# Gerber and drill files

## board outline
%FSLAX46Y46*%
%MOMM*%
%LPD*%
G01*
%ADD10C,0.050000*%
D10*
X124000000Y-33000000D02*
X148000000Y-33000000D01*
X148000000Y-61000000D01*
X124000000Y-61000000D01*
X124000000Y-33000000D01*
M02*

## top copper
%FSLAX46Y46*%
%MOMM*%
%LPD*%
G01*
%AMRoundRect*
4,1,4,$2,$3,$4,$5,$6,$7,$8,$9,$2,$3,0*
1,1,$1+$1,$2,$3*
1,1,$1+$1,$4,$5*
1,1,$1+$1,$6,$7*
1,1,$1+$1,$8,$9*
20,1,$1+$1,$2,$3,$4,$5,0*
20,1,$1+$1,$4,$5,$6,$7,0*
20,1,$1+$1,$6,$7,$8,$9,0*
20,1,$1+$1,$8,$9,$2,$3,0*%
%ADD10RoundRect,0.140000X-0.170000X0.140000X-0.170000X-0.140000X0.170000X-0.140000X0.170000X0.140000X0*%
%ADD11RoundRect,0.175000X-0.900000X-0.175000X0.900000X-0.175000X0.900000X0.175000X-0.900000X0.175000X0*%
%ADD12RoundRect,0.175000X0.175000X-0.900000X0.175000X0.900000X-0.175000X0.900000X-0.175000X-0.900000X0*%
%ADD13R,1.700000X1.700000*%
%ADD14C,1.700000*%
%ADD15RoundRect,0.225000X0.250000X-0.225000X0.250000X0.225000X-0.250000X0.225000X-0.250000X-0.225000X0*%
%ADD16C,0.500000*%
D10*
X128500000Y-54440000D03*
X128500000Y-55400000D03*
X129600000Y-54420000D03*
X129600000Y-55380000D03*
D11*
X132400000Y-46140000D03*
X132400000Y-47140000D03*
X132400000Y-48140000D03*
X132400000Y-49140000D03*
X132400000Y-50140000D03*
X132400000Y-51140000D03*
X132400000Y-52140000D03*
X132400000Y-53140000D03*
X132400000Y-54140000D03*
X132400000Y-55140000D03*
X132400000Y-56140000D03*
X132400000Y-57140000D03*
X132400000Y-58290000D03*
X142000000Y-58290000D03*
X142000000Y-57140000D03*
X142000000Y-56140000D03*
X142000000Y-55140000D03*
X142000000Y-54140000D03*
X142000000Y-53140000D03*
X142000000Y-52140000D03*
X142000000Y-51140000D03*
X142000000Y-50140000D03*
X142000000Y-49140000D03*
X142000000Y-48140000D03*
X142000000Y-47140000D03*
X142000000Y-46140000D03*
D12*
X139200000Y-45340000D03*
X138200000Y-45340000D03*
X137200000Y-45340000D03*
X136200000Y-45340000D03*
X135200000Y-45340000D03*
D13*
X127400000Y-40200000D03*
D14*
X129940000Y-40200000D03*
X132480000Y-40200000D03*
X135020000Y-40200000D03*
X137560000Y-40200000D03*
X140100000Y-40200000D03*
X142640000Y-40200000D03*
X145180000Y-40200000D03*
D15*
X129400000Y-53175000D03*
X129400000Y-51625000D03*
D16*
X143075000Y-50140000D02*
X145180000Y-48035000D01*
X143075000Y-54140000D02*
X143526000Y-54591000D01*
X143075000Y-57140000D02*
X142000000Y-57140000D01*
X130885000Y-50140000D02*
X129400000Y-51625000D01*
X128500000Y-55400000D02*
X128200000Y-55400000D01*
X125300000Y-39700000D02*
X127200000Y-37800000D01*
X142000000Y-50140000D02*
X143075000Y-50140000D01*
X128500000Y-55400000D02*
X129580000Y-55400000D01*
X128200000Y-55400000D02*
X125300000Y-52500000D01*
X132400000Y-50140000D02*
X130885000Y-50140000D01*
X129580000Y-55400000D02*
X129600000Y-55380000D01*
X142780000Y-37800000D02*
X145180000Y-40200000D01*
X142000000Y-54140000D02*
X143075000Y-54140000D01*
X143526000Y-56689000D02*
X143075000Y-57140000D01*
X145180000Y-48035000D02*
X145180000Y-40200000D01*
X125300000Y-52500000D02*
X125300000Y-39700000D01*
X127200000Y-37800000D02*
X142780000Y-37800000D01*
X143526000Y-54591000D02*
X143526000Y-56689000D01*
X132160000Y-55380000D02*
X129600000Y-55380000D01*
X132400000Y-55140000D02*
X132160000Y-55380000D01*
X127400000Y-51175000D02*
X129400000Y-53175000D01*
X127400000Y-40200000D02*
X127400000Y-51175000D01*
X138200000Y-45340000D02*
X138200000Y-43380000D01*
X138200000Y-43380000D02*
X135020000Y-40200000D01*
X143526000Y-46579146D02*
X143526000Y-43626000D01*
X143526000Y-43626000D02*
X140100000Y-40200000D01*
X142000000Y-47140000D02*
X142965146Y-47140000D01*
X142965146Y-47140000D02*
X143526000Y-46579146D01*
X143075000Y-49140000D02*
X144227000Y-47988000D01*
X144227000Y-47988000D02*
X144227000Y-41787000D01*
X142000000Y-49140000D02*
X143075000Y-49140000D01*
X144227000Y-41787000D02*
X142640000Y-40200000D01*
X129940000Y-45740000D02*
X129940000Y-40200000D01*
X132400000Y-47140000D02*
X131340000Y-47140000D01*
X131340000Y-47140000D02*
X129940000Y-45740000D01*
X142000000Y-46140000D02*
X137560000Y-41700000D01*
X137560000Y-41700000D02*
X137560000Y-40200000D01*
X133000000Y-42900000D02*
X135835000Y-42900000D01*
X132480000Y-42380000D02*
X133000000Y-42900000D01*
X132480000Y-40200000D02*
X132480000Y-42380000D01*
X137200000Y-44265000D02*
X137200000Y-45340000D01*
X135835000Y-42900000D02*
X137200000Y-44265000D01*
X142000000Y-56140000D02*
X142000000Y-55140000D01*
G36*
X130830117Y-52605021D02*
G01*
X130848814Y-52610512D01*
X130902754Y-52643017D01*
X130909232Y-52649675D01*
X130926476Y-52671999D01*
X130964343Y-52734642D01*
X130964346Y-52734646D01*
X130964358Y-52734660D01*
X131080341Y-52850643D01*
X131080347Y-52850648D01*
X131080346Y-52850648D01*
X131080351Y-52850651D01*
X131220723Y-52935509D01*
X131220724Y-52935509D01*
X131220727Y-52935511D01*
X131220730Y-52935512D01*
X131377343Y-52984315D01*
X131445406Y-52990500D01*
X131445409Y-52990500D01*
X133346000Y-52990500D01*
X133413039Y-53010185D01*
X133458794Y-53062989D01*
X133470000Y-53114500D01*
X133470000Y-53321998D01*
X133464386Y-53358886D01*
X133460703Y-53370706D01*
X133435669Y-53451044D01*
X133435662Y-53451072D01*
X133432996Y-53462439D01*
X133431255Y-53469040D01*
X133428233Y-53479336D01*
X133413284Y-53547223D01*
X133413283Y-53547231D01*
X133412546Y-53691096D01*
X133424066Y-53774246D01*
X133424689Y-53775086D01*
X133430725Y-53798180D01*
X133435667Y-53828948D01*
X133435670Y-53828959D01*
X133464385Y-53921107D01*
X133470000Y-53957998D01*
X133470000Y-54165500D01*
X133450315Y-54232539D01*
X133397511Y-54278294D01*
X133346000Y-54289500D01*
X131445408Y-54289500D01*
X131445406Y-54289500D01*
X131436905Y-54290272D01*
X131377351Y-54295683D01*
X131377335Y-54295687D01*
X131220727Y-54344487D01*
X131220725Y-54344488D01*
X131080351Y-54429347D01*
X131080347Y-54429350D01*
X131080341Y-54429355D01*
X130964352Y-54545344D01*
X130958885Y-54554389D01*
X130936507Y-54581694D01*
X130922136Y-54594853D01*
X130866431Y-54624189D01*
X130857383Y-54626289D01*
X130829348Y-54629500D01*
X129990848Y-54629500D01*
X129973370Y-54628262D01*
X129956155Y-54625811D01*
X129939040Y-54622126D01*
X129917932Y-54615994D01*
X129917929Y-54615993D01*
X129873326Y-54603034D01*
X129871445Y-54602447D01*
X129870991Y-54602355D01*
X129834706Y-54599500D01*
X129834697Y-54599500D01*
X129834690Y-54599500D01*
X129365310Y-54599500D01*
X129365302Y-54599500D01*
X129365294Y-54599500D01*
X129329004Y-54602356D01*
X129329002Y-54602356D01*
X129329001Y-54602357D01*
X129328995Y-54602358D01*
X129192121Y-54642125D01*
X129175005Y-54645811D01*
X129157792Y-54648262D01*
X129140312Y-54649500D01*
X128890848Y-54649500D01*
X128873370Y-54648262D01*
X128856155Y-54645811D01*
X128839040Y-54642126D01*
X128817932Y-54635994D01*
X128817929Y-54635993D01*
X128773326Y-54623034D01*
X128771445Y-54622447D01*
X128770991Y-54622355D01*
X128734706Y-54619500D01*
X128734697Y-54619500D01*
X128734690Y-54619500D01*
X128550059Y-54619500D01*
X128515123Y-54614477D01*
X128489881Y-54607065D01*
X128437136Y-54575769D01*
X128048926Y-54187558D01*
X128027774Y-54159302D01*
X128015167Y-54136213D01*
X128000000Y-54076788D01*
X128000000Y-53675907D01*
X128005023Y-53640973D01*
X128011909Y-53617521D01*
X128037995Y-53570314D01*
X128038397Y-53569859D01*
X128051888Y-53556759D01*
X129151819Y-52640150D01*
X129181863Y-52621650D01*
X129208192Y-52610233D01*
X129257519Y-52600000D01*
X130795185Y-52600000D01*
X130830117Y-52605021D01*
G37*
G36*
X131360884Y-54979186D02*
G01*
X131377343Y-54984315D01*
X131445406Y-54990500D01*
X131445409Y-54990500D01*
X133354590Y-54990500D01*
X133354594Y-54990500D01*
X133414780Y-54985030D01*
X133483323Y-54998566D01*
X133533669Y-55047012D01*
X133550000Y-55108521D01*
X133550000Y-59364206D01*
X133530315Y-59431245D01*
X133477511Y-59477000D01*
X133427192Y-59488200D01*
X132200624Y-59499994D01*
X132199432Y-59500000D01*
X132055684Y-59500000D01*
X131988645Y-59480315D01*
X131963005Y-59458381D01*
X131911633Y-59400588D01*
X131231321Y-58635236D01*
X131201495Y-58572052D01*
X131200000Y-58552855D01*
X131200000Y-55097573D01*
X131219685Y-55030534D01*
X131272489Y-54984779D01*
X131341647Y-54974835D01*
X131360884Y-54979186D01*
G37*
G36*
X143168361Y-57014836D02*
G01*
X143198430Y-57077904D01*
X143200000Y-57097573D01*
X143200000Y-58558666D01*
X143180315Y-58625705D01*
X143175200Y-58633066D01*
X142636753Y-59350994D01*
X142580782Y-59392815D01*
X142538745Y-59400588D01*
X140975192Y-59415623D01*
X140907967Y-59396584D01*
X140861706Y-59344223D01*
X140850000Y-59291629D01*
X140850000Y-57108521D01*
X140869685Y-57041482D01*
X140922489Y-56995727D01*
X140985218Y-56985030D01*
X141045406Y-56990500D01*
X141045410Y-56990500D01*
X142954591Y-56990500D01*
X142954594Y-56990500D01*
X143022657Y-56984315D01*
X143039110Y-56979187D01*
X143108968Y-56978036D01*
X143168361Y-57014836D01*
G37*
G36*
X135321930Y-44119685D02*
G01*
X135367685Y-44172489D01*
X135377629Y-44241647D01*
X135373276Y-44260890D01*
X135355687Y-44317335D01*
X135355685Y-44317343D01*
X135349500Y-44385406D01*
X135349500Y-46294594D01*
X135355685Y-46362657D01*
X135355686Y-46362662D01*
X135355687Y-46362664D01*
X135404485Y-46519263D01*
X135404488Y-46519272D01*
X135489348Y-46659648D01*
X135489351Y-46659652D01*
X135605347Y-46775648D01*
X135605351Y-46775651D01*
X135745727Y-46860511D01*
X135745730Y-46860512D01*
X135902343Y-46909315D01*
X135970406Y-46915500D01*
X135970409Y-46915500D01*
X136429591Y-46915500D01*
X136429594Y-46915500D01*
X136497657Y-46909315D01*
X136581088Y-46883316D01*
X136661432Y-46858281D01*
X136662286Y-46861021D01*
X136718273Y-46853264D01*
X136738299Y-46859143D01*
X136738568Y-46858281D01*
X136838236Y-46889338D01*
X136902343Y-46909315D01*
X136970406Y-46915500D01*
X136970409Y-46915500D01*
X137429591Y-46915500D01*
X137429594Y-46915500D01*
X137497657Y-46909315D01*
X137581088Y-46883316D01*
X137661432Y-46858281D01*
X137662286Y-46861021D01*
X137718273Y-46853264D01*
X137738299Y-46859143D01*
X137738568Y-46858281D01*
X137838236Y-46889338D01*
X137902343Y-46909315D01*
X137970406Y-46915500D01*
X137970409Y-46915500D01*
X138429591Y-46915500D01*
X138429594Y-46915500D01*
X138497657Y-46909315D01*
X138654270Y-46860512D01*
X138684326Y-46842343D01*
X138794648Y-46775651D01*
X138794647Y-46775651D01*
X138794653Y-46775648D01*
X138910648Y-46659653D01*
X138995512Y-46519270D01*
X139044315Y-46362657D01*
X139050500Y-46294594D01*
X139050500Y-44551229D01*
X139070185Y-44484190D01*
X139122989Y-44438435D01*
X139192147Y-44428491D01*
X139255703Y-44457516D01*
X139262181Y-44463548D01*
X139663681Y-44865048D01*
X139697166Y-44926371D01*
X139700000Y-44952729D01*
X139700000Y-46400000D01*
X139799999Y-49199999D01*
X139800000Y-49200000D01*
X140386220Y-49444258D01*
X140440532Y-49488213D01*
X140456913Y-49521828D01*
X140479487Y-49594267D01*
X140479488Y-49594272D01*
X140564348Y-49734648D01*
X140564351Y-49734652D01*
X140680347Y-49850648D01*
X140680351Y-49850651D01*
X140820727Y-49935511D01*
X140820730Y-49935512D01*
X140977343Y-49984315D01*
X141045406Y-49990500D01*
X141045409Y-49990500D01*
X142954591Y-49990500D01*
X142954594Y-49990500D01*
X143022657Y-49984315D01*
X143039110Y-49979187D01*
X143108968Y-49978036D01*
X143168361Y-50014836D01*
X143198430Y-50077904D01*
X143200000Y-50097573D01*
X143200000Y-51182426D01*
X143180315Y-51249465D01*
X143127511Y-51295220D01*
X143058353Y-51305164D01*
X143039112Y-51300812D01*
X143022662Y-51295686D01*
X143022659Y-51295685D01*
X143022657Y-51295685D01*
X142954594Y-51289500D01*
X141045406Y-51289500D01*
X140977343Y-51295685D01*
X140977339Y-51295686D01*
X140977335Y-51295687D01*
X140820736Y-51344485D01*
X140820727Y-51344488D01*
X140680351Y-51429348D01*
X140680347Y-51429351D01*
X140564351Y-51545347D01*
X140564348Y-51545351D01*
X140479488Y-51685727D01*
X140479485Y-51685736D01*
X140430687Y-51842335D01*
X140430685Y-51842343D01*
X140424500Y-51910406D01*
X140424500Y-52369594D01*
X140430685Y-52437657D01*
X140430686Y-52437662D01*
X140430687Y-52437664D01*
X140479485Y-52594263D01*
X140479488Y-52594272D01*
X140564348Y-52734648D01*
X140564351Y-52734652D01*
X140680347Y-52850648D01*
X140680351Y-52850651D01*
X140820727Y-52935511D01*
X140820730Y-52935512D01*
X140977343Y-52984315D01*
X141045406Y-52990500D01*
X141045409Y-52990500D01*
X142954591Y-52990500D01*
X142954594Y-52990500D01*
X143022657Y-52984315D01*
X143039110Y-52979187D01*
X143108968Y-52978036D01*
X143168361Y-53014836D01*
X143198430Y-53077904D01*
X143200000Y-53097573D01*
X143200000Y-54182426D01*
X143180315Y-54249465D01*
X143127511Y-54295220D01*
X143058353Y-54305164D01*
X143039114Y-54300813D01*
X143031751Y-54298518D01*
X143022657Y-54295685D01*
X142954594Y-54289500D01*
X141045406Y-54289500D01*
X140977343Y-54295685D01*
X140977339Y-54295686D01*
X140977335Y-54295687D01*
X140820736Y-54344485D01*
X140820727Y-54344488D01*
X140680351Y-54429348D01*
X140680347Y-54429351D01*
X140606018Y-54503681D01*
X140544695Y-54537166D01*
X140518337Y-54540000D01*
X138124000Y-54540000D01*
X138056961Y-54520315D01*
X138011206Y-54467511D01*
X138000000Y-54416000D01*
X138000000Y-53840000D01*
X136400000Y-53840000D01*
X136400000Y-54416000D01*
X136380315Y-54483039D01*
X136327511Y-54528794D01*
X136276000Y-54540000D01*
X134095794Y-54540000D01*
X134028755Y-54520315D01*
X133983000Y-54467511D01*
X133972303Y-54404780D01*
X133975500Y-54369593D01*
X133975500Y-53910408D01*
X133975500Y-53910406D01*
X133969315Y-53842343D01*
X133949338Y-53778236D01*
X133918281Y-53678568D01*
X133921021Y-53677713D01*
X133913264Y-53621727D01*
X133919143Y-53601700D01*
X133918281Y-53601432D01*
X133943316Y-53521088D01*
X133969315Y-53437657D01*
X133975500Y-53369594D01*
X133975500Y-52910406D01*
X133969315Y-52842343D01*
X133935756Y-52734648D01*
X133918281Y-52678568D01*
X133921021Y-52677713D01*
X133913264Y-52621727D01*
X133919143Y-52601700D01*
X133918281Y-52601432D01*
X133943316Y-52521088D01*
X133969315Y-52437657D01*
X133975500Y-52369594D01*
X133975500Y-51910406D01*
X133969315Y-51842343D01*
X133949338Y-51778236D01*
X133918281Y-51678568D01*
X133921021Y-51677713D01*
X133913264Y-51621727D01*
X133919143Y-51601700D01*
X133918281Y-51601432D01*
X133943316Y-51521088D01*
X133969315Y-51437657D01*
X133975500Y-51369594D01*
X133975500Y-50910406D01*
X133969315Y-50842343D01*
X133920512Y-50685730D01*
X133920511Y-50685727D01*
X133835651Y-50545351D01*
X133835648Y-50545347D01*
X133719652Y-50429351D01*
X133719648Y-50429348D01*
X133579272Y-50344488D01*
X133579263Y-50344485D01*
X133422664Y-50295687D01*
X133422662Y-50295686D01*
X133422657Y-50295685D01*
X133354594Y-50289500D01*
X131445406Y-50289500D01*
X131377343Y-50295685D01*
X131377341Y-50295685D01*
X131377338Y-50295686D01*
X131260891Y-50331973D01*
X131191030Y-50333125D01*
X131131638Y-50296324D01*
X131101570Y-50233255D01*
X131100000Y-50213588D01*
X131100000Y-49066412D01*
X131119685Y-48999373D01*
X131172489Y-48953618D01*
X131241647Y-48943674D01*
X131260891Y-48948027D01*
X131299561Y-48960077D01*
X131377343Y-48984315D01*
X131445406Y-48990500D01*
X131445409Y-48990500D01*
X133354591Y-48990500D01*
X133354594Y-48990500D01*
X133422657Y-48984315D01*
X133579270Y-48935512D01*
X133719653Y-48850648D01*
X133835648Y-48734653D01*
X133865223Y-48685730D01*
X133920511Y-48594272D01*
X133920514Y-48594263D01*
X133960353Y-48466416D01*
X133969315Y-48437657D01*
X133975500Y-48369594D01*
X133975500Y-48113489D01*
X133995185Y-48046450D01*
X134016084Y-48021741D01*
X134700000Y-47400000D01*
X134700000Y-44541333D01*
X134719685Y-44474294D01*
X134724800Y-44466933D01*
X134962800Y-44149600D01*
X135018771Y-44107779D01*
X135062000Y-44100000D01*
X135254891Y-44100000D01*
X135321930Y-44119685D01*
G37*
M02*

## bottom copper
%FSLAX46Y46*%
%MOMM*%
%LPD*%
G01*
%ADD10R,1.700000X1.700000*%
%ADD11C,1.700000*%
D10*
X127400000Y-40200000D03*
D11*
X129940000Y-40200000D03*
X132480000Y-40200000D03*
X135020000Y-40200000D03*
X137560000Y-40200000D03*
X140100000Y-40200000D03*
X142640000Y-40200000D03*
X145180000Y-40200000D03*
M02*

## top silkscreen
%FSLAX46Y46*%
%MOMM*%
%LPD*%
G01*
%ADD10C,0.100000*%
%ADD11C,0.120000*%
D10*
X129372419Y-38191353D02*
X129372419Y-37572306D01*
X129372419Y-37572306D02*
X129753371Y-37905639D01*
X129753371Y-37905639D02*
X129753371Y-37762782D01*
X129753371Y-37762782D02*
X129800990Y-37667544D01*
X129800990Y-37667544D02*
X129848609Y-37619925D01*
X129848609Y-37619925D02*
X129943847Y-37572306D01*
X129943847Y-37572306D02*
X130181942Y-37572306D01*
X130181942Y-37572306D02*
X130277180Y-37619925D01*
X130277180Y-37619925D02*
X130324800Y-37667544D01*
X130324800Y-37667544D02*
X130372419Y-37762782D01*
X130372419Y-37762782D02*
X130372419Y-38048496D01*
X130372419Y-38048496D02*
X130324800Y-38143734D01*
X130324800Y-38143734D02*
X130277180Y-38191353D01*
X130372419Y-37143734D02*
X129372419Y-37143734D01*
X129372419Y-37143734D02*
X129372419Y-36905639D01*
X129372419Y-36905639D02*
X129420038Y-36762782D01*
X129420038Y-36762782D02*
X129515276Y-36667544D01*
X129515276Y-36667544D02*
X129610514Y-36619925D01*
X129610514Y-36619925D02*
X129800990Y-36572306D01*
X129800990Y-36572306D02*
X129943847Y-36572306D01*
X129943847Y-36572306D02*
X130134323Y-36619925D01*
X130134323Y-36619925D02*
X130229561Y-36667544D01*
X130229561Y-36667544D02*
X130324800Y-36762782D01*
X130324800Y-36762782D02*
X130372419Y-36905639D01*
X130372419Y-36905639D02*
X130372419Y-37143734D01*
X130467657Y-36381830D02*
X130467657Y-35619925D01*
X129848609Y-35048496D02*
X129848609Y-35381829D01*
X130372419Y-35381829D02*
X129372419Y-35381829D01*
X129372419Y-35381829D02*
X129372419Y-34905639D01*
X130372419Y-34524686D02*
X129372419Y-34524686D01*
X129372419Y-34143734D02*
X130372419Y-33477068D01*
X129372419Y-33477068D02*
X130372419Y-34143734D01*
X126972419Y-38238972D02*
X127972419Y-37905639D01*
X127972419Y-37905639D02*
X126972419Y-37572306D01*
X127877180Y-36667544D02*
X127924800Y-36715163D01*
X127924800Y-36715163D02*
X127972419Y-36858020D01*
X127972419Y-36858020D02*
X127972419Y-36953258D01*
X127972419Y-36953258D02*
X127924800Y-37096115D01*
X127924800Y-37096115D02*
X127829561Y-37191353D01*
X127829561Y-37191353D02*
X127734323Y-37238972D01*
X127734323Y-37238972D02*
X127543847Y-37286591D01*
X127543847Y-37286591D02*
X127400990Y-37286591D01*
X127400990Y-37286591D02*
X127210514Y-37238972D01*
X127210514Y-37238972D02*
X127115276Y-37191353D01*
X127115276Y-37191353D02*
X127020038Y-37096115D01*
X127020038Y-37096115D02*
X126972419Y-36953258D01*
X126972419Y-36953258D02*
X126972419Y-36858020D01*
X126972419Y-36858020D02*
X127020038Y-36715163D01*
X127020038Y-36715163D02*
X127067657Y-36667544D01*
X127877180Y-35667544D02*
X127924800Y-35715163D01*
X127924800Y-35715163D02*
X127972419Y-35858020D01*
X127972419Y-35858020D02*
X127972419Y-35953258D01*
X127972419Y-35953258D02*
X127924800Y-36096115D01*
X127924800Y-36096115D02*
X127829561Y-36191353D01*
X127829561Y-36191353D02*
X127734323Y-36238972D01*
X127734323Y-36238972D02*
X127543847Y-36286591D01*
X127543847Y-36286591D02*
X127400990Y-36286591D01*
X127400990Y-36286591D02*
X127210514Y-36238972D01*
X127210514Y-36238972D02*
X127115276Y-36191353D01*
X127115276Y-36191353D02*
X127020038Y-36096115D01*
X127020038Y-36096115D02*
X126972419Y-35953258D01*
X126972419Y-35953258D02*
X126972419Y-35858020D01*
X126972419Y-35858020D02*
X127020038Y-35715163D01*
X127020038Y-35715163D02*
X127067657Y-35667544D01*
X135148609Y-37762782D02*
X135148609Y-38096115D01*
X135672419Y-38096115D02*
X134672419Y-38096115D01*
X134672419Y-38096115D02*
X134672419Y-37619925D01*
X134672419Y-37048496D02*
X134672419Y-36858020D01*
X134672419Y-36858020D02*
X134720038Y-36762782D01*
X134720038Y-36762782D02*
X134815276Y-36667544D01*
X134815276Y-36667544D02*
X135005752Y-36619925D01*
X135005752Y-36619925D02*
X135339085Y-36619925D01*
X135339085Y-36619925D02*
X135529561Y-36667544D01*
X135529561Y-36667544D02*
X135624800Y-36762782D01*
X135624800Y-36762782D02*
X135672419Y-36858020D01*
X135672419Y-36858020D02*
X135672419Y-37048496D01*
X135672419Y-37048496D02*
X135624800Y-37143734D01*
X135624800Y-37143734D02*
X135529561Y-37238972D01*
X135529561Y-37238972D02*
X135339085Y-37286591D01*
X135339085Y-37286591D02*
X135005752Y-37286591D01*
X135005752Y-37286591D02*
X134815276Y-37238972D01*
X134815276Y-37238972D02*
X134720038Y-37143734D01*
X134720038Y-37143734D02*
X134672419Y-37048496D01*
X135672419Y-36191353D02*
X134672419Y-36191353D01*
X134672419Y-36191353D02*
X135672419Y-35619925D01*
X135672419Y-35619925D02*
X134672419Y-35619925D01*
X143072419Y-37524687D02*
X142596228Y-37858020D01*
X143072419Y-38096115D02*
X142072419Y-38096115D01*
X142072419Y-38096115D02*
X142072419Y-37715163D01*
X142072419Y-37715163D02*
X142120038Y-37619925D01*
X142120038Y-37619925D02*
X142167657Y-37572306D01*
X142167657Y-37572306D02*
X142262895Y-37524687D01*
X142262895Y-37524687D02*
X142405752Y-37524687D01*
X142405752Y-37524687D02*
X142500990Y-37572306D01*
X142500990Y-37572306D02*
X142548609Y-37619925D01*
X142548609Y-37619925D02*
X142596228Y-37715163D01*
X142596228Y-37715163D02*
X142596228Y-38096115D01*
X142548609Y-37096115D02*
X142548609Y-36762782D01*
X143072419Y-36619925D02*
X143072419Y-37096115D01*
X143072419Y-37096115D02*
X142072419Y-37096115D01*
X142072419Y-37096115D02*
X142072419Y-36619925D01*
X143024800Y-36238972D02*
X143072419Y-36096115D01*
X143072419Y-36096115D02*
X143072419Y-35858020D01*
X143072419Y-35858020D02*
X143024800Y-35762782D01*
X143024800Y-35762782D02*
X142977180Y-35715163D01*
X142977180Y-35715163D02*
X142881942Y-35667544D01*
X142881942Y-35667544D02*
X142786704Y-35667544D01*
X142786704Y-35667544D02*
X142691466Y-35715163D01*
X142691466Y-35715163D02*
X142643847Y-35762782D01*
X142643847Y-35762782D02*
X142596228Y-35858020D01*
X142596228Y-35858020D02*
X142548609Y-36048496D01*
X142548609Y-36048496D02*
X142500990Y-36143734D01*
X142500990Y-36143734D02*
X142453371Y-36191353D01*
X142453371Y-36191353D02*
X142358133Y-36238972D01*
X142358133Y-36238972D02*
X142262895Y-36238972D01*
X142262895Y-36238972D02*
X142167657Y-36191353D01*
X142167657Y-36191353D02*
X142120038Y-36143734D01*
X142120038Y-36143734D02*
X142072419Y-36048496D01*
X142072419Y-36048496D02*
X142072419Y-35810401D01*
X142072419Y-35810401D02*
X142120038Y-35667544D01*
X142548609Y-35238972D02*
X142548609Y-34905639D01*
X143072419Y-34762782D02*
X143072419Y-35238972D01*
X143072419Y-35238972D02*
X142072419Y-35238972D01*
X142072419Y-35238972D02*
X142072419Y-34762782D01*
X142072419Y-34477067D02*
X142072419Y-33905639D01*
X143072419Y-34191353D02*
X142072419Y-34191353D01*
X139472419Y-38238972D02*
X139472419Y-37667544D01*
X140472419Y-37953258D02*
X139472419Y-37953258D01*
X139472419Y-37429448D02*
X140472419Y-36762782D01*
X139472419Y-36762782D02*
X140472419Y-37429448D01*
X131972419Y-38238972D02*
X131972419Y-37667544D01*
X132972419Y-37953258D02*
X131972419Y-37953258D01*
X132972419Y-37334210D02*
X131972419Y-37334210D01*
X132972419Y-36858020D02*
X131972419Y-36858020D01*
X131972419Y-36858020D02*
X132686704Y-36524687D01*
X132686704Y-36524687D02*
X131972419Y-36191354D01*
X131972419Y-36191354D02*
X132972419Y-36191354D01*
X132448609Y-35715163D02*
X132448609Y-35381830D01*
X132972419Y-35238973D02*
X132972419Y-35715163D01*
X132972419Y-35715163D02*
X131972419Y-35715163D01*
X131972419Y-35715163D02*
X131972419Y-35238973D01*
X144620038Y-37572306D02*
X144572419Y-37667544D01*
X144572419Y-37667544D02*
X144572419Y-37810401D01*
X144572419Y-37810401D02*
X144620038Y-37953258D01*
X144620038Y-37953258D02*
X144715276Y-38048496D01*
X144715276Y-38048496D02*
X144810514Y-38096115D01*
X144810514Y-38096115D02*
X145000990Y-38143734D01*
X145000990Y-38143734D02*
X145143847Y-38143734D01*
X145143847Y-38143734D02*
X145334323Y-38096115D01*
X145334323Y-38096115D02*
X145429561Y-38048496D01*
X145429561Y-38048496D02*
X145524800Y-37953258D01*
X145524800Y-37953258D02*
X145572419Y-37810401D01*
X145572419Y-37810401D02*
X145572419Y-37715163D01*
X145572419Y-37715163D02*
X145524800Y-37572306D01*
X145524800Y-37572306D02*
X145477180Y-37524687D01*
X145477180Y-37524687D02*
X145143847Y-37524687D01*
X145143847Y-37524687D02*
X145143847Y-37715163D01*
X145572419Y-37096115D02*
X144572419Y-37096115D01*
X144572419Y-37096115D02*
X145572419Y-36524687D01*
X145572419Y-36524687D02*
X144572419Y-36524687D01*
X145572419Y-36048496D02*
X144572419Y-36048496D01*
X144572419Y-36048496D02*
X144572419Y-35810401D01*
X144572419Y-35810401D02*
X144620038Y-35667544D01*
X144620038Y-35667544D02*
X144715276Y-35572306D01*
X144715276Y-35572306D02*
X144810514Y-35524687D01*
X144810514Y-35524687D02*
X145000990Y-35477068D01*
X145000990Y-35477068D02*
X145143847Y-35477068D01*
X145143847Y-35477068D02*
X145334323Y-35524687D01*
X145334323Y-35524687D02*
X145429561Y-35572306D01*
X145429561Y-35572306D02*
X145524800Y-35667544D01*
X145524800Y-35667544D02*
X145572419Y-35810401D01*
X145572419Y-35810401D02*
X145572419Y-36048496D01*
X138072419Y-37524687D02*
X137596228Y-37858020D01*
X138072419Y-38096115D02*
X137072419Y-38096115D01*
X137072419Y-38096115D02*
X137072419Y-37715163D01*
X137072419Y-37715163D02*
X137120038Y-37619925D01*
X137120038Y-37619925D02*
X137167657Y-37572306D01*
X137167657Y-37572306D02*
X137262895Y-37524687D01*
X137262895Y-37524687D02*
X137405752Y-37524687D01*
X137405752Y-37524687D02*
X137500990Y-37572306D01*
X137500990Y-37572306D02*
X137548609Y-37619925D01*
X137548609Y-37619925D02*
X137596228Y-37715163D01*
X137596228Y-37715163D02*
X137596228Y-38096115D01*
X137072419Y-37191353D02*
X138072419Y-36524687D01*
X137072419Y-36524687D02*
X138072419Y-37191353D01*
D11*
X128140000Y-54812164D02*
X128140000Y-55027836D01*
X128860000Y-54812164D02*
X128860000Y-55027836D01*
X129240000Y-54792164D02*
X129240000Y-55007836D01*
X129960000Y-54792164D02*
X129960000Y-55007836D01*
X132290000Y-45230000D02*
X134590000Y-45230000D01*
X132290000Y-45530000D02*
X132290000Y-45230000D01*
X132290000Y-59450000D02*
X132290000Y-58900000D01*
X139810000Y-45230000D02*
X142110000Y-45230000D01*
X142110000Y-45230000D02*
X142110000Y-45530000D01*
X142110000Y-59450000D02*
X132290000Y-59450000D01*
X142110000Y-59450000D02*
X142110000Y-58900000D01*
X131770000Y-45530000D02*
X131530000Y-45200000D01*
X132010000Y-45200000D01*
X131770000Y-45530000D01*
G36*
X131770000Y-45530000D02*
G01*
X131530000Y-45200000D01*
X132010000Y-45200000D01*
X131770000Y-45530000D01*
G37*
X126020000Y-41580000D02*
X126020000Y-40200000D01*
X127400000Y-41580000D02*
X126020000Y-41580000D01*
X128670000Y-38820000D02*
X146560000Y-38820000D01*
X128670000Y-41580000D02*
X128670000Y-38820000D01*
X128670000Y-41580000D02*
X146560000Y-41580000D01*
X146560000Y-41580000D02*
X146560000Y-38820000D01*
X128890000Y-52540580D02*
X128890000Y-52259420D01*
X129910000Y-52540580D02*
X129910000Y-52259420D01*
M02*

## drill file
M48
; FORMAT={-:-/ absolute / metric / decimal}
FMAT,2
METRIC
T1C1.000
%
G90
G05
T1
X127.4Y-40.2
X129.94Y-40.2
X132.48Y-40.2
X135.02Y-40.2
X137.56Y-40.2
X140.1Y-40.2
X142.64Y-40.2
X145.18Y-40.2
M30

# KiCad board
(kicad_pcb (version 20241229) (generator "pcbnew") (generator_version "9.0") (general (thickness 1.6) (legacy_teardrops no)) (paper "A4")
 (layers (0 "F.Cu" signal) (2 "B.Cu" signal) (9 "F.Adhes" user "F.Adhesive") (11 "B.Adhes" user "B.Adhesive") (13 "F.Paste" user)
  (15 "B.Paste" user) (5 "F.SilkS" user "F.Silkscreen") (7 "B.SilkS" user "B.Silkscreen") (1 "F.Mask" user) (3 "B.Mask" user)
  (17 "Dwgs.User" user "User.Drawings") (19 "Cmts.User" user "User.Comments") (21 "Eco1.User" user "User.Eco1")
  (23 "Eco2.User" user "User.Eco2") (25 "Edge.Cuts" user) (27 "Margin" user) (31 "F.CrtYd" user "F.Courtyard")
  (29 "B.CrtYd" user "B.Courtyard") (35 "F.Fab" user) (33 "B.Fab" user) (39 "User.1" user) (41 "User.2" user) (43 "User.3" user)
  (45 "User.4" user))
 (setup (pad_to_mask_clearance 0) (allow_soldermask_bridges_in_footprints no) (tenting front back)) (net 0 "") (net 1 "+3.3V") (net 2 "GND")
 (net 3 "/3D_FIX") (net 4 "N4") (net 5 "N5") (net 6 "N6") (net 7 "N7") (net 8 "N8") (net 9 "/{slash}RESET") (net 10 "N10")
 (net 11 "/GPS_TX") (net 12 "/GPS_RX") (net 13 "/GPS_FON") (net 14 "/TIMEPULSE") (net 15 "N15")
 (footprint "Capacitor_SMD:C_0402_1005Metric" (layer "F.Cu") (at 128.5 54.92 -90)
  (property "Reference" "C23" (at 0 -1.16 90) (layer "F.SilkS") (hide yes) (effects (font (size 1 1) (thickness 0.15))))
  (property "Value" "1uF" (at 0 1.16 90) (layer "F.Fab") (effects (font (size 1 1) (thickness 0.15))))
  (fp_line (start -0.107836 0.36) (end 0.107836 0.36) (stroke (width 0.12) (type solid)) (layer "F.SilkS"))
  (fp_line (start -0.107836 -0.36) (end 0.107836 -0.36) (stroke (width 0.12) (type solid)) (layer "F.SilkS"))
  (pad "1" smd roundrect (at -0.48 0 270) (size 0.56 0.62) (layers "F.Cu" "F.Mask" "F.Paste") (roundrect_rratio 0.25) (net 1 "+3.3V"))
  (pad "2" smd roundrect (at 0.48 0 270) (size 0.56 0.62) (layers "F.Cu" "F.Mask" "F.Paste") (roundrect_rratio 0.25) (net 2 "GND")))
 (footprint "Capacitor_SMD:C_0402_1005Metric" (layer "F.Cu") (at 129.6 54.9 -90)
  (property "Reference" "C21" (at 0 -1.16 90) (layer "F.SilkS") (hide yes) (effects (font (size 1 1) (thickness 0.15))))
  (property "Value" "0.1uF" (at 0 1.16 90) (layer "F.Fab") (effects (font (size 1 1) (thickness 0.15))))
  (fp_line (start -0.107836 0.36) (end 0.107836 0.36) (stroke (width 0.12) (type solid)) (layer "F.SilkS"))
  (fp_line (start -0.107836 -0.36) (end 0.107836 -0.36) (stroke (width 0.12) (type solid)) (layer "F.SilkS"))
  (pad "1" smd roundrect (at -0.48 0 270) (size 0.56 0.62) (layers "F.Cu" "F.Mask" "F.Paste") (roundrect_rratio 0.25) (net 1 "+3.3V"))
  (pad "2" smd roundrect (at 0.48 0 270) (size 0.56 0.62) (layers "F.Cu" "F.Mask" "F.Paste") (roundrect_rratio 0.25) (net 2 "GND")))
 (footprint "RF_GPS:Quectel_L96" (layer "F.Cu") (at 137.2 52.34)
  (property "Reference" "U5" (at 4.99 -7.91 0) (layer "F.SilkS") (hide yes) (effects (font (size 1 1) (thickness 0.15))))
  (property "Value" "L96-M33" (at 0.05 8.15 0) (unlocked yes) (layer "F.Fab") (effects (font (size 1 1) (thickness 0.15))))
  (fp_line (start -4.91 -7.11) (end -2.61 -7.11) (stroke (width 0.12) (type default)) (layer "F.SilkS"))
  (fp_line (start -4.91 -6.81) (end -4.91 -7.11) (stroke (width 0.12) (type default)) (layer "F.SilkS"))
  (fp_line (start -4.91 7.11) (end -4.91 6.56) (stroke (width 0.12) (type default)) (layer "F.SilkS"))
  (fp_line (start 2.61 -7.11) (end 4.91 -7.11) (stroke (width 0.12) (type default)) (layer "F.SilkS"))
  (fp_line (start 4.91 -7.11) (end 4.91 -6.81) (stroke (width 0.12) (type default)) (layer "F.SilkS"))
  (fp_line (start 4.91 7.11) (end -4.91 7.11) (stroke (width 0.12) (type default)) (layer "F.SilkS"))
  (fp_line (start 4.91 7.11) (end 4.91 6.56) (stroke (width 0.12) (type default)) (layer "F.SilkS"))
  (fp_poly
   (pts (xy -5.43 -6.81) (xy -5.67 -7.14) (xy -5.19 -7.14) (xy -5.43 -6.81)) (stroke (width 0.12) (type solid)) (fill yes) (layer "F.SilkS"))
  (pad "1" smd roundrect (at -4.8 -6.2) (size 2.15 0.7) (layers "F.Cu" "F.Mask" "F.Paste") (roundrect_rratio 0.25) (thermal_bridge_angle 45))
  (pad "2" smd roundrect (at -4.8 -5.2) (size 2.15 0.7) (layers "F.Cu" "F.Mask" "F.Paste") (roundrect_rratio 0.25) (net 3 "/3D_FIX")
   (thermal_bridge_angle 45))
  (pad "3" smd roundrect (at -4.8 -4.2) (size 2.15 0.7) (layers "F.Cu" "F.Mask" "F.Paste") (roundrect_rratio 0.25) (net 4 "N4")
   (thermal_bridge_angle 45))
  (pad "4" smd roundrect (at -4.8 -3.2) (size 2.15 0.7) (layers "F.Cu" "F.Mask" "F.Paste") (roundrect_rratio 0.25) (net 2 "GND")
   (thermal_bridge_angle 45))
  (pad "5" smd roundrect (at -4.8 -2.2) (size 2.15 0.7) (layers "F.Cu" "F.Mask" "F.Paste") (roundrect_rratio 0.25) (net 2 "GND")
   (thermal_bridge_angle 45))
  (pad "6" smd roundrect (at -4.8 -1.2) (size 2.15 0.7) (layers "F.Cu" "F.Mask" "F.Paste") (roundrect_rratio 0.25) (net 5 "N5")
   (thermal_bridge_angle 45))
  (pad "7" smd roundrect (at -4.8 -0.2) (size 2.15 0.7) (layers "F.Cu" "F.Mask" "F.Paste") (roundrect_rratio 0.25) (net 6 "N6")
   (thermal_bridge_angle 45))
  (pad "8" smd roundrect (at -4.8 0.8) (size 2.15 0.7) (layers "F.Cu" "F.Mask" "F.Paste") (roundrect_rratio 0.25) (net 1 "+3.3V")
   (thermal_bridge_angle 45))
  (pad "9" smd roundrect (at -4.8 1.8) (size 2.15 0.7) (layers "F.Cu" "F.Mask" "F.Paste") (roundrect_rratio 0.25) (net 1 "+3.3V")
   (thermal_bridge_angle 45))
  (pad "10" smd roundrect (at -4.8 2.8) (size 2.15 0.7) (layers "F.Cu" "F.Mask" "F.Paste") (roundrect_rratio 0.25) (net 2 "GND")
   (thermal_bridge_angle 45))
  (pad "11" smd roundrect (at -4.8 3.8) (size 2.15 0.7) (layers "F.Cu" "F.Mask" "F.Paste") (roundrect_rratio 0.25) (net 2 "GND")
   (thermal_bridge_angle 45))
  (pad "12" smd roundrect (at -4.8 4.8) (size 2.15 0.7) (layers "F.Cu" "F.Mask" "F.Paste") (roundrect_rratio 0.25) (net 2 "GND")
   (thermal_bridge_angle 45))
  (pad "13" smd roundrect (at -4.8 5.95) (size 2.15 0.7) (layers "F.Cu" "F.Mask" "F.Paste") (roundrect_rratio 0.25) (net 2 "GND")
   (thermal_bridge_angle 45))
  (pad "14" smd roundrect (at 4.8 5.95) (size 2.15 0.7) (layers "F.Cu" "F.Mask" "F.Paste") (roundrect_rratio 0.25) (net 2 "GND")
   (thermal_bridge_angle 45))
  (pad "15" smd roundrect (at 4.8 4.8) (size 2.15 0.7) (layers "F.Cu" "F.Mask" "F.Paste") (roundrect_rratio 0.25) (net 2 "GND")
   (thermal_bridge_angle 45))
  (pad "16" smd roundrect (at 4.8 3.8) (size 2.15 0.7) (layers "F.Cu" "F.Mask" "F.Paste") (roundrect_rratio 0.25) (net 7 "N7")
   (thermal_bridge_angle 45))
  (pad "17" smd roundrect (at 4.8 2.8) (size 2.15 0.7) (layers "F.Cu" "F.Mask" "F.Paste") (roundrect_rratio 0.25) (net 7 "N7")
   (thermal_bridge_angle 45))
  (pad "18" smd roundrect (at 4.8 1.8) (size 2.15 0.7) (layers "F.Cu" "F.Mask" "F.Paste") (roundrect_rratio 0.25) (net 2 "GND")
   (thermal_bridge_angle 45))
  (pad "19" smd roundrect (at 4.8 0.8) (size 2.15 0.7) (layers "F.Cu" "F.Mask" "F.Paste") (roundrect_rratio 0.25) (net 2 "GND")
   (thermal_bridge_angle 45))
  (pad "20" smd roundrect (at 4.8 -0.2) (size 2.15 0.7) (layers "F.Cu" "F.Mask" "F.Paste") (roundrect_rratio 0.25) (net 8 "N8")
   (thermal_bridge_angle 45))
  (pad "21" smd roundrect (at 4.8 -1.2) (size 2.15 0.7) (layers "F.Cu" "F.Mask" "F.Paste") (roundrect_rratio 0.25) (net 2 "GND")
   (thermal_bridge_angle 45))
  (pad "22" smd roundrect (at 4.8 -2.2) (size 2.15 0.7) (layers "F.Cu" "F.Mask" "F.Paste") (roundrect_rratio 0.25) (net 2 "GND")
   (thermal_bridge_angle 45))
  (pad "23" smd roundrect (at 4.8 -3.2) (size 2.15 0.7) (layers "F.Cu" "F.Mask" "F.Paste") (roundrect_rratio 0.25) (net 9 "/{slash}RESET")
   (thermal_bridge_angle 45))
  (pad "24" smd roundrect (at 4.8 -4.2) (size 2.15 0.7) (layers "F.Cu" "F.Mask" "F.Paste") (roundrect_rratio 0.25) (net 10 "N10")
   (thermal_bridge_angle 45))
  (pad "25" smd roundrect (at 4.8 -5.2) (size 2.15 0.7) (layers "F.Cu" "F.Mask" "F.Paste") (roundrect_rratio 0.25) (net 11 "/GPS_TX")
   (thermal_bridge_angle 45))
  (pad "26" smd roundrect (at 4.8 -6.2) (size 2.15 0.7) (layers "F.Cu" "F.Mask" "F.Paste") (roundrect_rratio 0.25) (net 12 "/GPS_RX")
   (thermal_bridge_angle 45))
  (pad "27" smd roundrect (at 2 -7 90) (size 2.15 0.7) (layers "F.Cu" "F.Mask" "F.Paste") (roundrect_rratio 0.25) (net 2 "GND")
   (thermal_bridge_angle 45))
  (pad "28" smd roundrect (at 1 -7 90) (size 2.15 0.7) (layers "F.Cu" "F.Mask" "F.Paste") (roundrect_rratio 0.25) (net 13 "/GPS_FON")
   (thermal_bridge_angle 45))
  (pad "29" smd roundrect (at 0 -7 90) (size 2.15 0.7) (layers "F.Cu" "F.Mask" "F.Paste") (roundrect_rratio 0.25) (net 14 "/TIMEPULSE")
   (thermal_bridge_angle 45))
  (pad "30" smd roundrect (at -1 -7 90) (size 2.15 0.7) (layers "F.Cu" "F.Mask" "F.Paste") (roundrect_rratio 0.25) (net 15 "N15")
   (thermal_bridge_angle 45))
  (pad "31" smd roundrect (at -2 -7 90) (size 2.15 0.7) (layers "F.Cu" "F.Mask" "F.Paste") (roundrect_rratio 0.25) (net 2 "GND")
   (thermal_bridge_angle 45))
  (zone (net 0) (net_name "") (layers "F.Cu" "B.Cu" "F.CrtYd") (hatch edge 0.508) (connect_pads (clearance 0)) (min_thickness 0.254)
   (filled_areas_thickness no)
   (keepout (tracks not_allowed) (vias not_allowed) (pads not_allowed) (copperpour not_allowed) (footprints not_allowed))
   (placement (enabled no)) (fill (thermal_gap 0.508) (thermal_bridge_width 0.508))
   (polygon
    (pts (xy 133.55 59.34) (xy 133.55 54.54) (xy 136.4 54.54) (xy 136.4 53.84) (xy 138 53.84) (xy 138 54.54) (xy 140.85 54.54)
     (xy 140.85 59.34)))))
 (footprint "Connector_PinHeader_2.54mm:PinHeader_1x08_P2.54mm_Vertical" (layer "F.Cu") (at 127.4 40.2 90)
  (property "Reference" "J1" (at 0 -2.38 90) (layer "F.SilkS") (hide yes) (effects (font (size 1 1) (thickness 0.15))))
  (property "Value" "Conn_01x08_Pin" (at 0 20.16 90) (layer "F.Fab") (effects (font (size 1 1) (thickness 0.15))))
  (fp_line (start -1.38 -1.38) (end 0 -1.38) (stroke (width 0.12) (type solid)) (layer "F.SilkS"))
  (fp_line (start -1.38 0) (end -1.38 -1.38) (stroke (width 0.12) (type solid)) (layer "F.SilkS"))
  (fp_line (start 1.38 1.27) (end 1.38 19.16) (stroke (width 0.12) (type solid)) (layer "F.SilkS"))
  (fp_line (start -1.38 1.27) (end 1.38 1.27) (stroke (width 0.12) (type solid)) (layer "F.SilkS"))
  (fp_line (start -1.38 1.27) (end -1.38 19.16) (stroke (width 0.12) (type solid)) (layer "F.SilkS"))
  (fp_line (start -1.38 19.16) (end 1.38 19.16) (stroke (width 0.12) (type solid)) (layer "F.SilkS"))
  (pad "1" thru_hole rect (at 0 0 90) (size 1.7 1.7) (drill 1) (layers "*.Cu" "*.Mask") (remove_unused_layers no) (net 1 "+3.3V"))
  (pad "2" thru_hole circle (at 0 2.54 90) (size 1.7 1.7) (drill 1) (layers "*.Cu" "*.Mask") (remove_unused_layers no) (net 3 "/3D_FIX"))
  (pad "3" thru_hole circle (at 0 5.08 90) (size 1.7 1.7) (drill 1) (layers "*.Cu" "*.Mask") (remove_unused_layers no) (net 14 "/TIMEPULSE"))
  (pad "4" thru_hole circle (at 0 7.62 90) (size 1.7 1.7) (drill 1) (layers "*.Cu" "*.Mask") (remove_unused_layers no) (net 13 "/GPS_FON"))
  (pad "5" thru_hole circle (at 0 10.16 90) (size 1.7 1.7) (drill 1) (layers "*.Cu" "*.Mask") (remove_unused_layers no) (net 12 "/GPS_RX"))
  (pad "6" thru_hole circle (at 0 12.7 90) (size 1.7 1.7) (drill 1) (layers "*.Cu" "*.Mask") (remove_unused_layers no) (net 11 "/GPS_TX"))
  (pad "7" thru_hole circle (at 0 15.24 90) (size 1.7 1.7) (drill 1) (layers "*.Cu" "*.Mask") (remove_unused_layers no)
   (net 9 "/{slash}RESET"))
  (pad "8" thru_hole circle (at 0 17.78 90) (size 1.7 1.7) (drill 1) (layers "*.Cu" "*.Mask") (remove_unused_layers no) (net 2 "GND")))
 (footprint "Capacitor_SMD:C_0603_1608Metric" (layer "F.Cu") (at 129.4 52.4 90)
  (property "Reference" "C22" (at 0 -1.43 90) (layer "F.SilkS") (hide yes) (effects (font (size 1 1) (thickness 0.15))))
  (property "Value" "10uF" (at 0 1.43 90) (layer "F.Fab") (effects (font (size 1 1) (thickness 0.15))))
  (fp_line (start -0.14058 -0.51) (end 0.14058 -0.51) (stroke (width 0.12) (type solid)) (layer "F.SilkS"))
  (fp_line (start -0.14058 0.51) (end 0.14058 0.51) (stroke (width 0.12) (type solid)) (layer "F.SilkS"))
  (pad "1" smd roundrect (at -0.775 0 90) (size 0.9 0.95) (layers "F.Cu" "F.Mask" "F.Paste") (roundrect_rratio 0.25) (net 1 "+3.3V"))
  (pad "2" smd roundrect (at 0.775 0 90) (size 0.9 0.95) (layers "F.Cu" "F.Mask" "F.Paste") (roundrect_rratio 0.25) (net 2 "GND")))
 (gr_rect (start 124 33) (end 148 61) (stroke (width 0.05) (type default)) (fill no) (layer "Edge.Cuts"))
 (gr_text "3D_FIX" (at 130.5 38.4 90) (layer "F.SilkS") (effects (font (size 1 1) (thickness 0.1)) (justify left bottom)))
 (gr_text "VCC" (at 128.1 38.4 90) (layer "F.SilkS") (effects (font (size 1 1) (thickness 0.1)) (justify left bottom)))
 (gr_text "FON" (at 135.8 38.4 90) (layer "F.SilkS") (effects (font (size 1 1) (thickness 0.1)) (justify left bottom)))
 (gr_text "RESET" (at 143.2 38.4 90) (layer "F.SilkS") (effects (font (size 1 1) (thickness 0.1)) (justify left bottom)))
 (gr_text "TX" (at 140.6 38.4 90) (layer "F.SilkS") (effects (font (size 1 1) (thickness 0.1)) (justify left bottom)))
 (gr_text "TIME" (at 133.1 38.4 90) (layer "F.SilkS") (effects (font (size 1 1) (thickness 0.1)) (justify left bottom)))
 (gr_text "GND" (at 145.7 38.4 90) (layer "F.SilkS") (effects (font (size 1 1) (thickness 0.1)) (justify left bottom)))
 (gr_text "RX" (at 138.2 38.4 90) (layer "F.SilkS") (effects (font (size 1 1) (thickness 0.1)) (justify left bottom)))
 (segment (start 143.075 50.14) (end 145.18 48.035) (width 0.5) (layer "F.Cu") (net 2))
 (segment (start 143.075 54.14) (end 143.526 54.591) (width 0.5) (layer "F.Cu") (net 2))
 (segment (start 143.075 57.14) (end 142 57.14) (width 0.5) (layer "F.Cu") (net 2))
 (segment (start 130.885 50.14) (end 129.4 51.625) (width 0.5) (layer "F.Cu") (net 2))
 (segment (start 128.5 55.4) (end 128.2 55.4) (width 0.5) (layer "F.Cu") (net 2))
 (segment (start 125.3 39.7) (end 127.2 37.8) (width 0.5) (layer "F.Cu") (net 2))
 (segment (start 142 50.14) (end 143.075 50.14) (width 0.5) (layer "F.Cu") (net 2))
 (segment (start 128.5 55.4) (end 129.58 55.4) (width 0.5) (layer "F.Cu") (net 2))
 (segment (start 128.2 55.4) (end 125.3 52.5) (width 0.5) (layer "F.Cu") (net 2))
 (segment (start 132.4 50.14) (end 130.885 50.14) (width 0.5) (layer "F.Cu") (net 2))
 (segment (start 129.58 55.4) (end 129.6 55.38) (width 0.5) (layer "F.Cu") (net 2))
 (segment (start 142.78 37.8) (end 145.18 40.2) (width 0.5) (layer "F.Cu") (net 2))
 (segment (start 142 54.14) (end 143.075 54.14) (width 0.5) (layer "F.Cu") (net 2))
 (segment (start 143.526 56.689) (end 143.075 57.14) (width 0.5) (layer "F.Cu") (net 2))
 (segment (start 145.18 48.035) (end 145.18 40.2) (width 0.5) (layer "F.Cu") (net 2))
 (segment (start 125.3 52.5) (end 125.3 39.7) (width 0.5) (layer "F.Cu") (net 2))
 (segment (start 127.2 37.8) (end 142.78 37.8) (width 0.5) (layer "F.Cu") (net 2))
 (segment (start 143.526 54.591) (end 143.526 56.689) (width 0.5) (layer "F.Cu") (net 2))
 (segment (start 132.16 55.38) (end 129.6 55.38) (width 0.5) (layer "F.Cu") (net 2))
 (segment (start 132.4 55.14) (end 132.16 55.38) (width 0.5) (layer "F.Cu") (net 2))
 (segment (start 127.4 51.175) (end 129.4 53.175) (width 0.5) (layer "F.Cu") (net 1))
 (segment (start 127.4 40.2) (end 127.4 51.175) (width 0.5) (layer "F.Cu") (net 1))
 (segment (start 138.2 45.34) (end 138.2 43.38) (width 0.5) (layer "F.Cu") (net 13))
 (segment (start 138.2 43.38) (end 135.02 40.2) (width 0.5) (layer "F.Cu") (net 13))
 (segment (start 143.526 46.579146) (end 143.526 43.626) (width 0.5) (layer "F.Cu") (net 11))
 (segment (start 143.526 43.626) (end 140.1 40.2) (width 0.5) (layer "F.Cu") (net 11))
 (segment (start 142 47.14) (end 142.965146 47.14) (width 0.5) (layer "F.Cu") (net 11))
 (segment (start 142.965146 47.14) (end 143.526 46.579146) (width 0.5) (layer "F.Cu") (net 11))
 (segment (start 143.075 49.14) (end 144.227 47.988) (width 0.5) (layer "F.Cu") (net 9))
 (segment (start 144.227 47.988) (end 144.227 41.787) (width 0.5) (layer "F.Cu") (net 9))
 (segment (start 142 49.14) (end 143.075 49.14) (width 0.5) (layer "F.Cu") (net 9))
 (segment (start 144.227 41.787) (end 142.64 40.2) (width 0.5) (layer "F.Cu") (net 9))
 (segment (start 129.94 45.74) (end 129.94 40.2) (width 0.5) (layer "F.Cu") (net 3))
 (segment (start 132.4 47.14) (end 131.34 47.14) (width 0.5) (layer "F.Cu") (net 3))
 (segment (start 131.34 47.14) (end 129.94 45.74) (width 0.5) (layer "F.Cu") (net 3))
 (segment (start 142 46.14) (end 137.56 41.7) (width 0.5) (layer "F.Cu") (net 12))
 (segment (start 137.56 41.7) (end 137.56 40.2) (width 0.5) (layer "F.Cu") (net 12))
 (segment (start 133 42.9) (end 135.835 42.9) (width 0.5) (layer "F.Cu") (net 14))
 (segment (start 132.48 42.38) (end 133 42.9) (width 0.5) (layer "F.Cu") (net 14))
 (segment (start 132.48 40.2) (end 132.48 42.38) (width 0.5) (layer "F.Cu") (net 14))
 (segment (start 137.2 44.265) (end 137.2 45.34) (width 0.5) (layer "F.Cu") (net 14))
 (segment (start 135.835 42.9) (end 137.2 44.265) (width 0.5) (layer "F.Cu") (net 14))
 (segment (start 142 56.14) (end 142 55.14) (width 0.5) (layer "F.Cu") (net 7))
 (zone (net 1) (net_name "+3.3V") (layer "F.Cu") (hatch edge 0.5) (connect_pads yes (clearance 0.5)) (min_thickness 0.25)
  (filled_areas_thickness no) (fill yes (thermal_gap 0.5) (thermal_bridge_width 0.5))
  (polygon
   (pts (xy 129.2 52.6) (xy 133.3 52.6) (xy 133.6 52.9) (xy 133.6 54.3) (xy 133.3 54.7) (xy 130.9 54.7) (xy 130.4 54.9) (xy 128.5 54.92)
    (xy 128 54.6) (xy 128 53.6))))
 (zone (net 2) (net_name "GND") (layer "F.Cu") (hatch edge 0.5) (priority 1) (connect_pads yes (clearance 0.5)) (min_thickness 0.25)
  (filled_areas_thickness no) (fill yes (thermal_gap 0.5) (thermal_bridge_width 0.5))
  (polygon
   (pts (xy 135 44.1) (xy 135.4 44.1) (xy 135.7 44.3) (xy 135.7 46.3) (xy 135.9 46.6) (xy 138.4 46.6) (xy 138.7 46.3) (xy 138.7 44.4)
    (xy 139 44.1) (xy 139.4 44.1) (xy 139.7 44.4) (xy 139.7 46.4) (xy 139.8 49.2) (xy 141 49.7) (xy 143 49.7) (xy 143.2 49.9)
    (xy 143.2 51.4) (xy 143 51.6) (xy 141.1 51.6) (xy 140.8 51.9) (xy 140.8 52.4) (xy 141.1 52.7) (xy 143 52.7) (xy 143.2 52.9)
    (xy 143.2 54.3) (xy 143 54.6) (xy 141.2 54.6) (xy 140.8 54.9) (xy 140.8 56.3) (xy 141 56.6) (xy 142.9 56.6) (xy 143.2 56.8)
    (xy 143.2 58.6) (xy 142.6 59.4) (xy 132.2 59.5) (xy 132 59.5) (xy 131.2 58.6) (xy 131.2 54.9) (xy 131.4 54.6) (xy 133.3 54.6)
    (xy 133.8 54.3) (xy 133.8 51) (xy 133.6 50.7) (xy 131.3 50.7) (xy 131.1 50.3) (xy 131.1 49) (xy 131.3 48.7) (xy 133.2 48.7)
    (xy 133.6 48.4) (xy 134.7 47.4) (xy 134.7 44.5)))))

